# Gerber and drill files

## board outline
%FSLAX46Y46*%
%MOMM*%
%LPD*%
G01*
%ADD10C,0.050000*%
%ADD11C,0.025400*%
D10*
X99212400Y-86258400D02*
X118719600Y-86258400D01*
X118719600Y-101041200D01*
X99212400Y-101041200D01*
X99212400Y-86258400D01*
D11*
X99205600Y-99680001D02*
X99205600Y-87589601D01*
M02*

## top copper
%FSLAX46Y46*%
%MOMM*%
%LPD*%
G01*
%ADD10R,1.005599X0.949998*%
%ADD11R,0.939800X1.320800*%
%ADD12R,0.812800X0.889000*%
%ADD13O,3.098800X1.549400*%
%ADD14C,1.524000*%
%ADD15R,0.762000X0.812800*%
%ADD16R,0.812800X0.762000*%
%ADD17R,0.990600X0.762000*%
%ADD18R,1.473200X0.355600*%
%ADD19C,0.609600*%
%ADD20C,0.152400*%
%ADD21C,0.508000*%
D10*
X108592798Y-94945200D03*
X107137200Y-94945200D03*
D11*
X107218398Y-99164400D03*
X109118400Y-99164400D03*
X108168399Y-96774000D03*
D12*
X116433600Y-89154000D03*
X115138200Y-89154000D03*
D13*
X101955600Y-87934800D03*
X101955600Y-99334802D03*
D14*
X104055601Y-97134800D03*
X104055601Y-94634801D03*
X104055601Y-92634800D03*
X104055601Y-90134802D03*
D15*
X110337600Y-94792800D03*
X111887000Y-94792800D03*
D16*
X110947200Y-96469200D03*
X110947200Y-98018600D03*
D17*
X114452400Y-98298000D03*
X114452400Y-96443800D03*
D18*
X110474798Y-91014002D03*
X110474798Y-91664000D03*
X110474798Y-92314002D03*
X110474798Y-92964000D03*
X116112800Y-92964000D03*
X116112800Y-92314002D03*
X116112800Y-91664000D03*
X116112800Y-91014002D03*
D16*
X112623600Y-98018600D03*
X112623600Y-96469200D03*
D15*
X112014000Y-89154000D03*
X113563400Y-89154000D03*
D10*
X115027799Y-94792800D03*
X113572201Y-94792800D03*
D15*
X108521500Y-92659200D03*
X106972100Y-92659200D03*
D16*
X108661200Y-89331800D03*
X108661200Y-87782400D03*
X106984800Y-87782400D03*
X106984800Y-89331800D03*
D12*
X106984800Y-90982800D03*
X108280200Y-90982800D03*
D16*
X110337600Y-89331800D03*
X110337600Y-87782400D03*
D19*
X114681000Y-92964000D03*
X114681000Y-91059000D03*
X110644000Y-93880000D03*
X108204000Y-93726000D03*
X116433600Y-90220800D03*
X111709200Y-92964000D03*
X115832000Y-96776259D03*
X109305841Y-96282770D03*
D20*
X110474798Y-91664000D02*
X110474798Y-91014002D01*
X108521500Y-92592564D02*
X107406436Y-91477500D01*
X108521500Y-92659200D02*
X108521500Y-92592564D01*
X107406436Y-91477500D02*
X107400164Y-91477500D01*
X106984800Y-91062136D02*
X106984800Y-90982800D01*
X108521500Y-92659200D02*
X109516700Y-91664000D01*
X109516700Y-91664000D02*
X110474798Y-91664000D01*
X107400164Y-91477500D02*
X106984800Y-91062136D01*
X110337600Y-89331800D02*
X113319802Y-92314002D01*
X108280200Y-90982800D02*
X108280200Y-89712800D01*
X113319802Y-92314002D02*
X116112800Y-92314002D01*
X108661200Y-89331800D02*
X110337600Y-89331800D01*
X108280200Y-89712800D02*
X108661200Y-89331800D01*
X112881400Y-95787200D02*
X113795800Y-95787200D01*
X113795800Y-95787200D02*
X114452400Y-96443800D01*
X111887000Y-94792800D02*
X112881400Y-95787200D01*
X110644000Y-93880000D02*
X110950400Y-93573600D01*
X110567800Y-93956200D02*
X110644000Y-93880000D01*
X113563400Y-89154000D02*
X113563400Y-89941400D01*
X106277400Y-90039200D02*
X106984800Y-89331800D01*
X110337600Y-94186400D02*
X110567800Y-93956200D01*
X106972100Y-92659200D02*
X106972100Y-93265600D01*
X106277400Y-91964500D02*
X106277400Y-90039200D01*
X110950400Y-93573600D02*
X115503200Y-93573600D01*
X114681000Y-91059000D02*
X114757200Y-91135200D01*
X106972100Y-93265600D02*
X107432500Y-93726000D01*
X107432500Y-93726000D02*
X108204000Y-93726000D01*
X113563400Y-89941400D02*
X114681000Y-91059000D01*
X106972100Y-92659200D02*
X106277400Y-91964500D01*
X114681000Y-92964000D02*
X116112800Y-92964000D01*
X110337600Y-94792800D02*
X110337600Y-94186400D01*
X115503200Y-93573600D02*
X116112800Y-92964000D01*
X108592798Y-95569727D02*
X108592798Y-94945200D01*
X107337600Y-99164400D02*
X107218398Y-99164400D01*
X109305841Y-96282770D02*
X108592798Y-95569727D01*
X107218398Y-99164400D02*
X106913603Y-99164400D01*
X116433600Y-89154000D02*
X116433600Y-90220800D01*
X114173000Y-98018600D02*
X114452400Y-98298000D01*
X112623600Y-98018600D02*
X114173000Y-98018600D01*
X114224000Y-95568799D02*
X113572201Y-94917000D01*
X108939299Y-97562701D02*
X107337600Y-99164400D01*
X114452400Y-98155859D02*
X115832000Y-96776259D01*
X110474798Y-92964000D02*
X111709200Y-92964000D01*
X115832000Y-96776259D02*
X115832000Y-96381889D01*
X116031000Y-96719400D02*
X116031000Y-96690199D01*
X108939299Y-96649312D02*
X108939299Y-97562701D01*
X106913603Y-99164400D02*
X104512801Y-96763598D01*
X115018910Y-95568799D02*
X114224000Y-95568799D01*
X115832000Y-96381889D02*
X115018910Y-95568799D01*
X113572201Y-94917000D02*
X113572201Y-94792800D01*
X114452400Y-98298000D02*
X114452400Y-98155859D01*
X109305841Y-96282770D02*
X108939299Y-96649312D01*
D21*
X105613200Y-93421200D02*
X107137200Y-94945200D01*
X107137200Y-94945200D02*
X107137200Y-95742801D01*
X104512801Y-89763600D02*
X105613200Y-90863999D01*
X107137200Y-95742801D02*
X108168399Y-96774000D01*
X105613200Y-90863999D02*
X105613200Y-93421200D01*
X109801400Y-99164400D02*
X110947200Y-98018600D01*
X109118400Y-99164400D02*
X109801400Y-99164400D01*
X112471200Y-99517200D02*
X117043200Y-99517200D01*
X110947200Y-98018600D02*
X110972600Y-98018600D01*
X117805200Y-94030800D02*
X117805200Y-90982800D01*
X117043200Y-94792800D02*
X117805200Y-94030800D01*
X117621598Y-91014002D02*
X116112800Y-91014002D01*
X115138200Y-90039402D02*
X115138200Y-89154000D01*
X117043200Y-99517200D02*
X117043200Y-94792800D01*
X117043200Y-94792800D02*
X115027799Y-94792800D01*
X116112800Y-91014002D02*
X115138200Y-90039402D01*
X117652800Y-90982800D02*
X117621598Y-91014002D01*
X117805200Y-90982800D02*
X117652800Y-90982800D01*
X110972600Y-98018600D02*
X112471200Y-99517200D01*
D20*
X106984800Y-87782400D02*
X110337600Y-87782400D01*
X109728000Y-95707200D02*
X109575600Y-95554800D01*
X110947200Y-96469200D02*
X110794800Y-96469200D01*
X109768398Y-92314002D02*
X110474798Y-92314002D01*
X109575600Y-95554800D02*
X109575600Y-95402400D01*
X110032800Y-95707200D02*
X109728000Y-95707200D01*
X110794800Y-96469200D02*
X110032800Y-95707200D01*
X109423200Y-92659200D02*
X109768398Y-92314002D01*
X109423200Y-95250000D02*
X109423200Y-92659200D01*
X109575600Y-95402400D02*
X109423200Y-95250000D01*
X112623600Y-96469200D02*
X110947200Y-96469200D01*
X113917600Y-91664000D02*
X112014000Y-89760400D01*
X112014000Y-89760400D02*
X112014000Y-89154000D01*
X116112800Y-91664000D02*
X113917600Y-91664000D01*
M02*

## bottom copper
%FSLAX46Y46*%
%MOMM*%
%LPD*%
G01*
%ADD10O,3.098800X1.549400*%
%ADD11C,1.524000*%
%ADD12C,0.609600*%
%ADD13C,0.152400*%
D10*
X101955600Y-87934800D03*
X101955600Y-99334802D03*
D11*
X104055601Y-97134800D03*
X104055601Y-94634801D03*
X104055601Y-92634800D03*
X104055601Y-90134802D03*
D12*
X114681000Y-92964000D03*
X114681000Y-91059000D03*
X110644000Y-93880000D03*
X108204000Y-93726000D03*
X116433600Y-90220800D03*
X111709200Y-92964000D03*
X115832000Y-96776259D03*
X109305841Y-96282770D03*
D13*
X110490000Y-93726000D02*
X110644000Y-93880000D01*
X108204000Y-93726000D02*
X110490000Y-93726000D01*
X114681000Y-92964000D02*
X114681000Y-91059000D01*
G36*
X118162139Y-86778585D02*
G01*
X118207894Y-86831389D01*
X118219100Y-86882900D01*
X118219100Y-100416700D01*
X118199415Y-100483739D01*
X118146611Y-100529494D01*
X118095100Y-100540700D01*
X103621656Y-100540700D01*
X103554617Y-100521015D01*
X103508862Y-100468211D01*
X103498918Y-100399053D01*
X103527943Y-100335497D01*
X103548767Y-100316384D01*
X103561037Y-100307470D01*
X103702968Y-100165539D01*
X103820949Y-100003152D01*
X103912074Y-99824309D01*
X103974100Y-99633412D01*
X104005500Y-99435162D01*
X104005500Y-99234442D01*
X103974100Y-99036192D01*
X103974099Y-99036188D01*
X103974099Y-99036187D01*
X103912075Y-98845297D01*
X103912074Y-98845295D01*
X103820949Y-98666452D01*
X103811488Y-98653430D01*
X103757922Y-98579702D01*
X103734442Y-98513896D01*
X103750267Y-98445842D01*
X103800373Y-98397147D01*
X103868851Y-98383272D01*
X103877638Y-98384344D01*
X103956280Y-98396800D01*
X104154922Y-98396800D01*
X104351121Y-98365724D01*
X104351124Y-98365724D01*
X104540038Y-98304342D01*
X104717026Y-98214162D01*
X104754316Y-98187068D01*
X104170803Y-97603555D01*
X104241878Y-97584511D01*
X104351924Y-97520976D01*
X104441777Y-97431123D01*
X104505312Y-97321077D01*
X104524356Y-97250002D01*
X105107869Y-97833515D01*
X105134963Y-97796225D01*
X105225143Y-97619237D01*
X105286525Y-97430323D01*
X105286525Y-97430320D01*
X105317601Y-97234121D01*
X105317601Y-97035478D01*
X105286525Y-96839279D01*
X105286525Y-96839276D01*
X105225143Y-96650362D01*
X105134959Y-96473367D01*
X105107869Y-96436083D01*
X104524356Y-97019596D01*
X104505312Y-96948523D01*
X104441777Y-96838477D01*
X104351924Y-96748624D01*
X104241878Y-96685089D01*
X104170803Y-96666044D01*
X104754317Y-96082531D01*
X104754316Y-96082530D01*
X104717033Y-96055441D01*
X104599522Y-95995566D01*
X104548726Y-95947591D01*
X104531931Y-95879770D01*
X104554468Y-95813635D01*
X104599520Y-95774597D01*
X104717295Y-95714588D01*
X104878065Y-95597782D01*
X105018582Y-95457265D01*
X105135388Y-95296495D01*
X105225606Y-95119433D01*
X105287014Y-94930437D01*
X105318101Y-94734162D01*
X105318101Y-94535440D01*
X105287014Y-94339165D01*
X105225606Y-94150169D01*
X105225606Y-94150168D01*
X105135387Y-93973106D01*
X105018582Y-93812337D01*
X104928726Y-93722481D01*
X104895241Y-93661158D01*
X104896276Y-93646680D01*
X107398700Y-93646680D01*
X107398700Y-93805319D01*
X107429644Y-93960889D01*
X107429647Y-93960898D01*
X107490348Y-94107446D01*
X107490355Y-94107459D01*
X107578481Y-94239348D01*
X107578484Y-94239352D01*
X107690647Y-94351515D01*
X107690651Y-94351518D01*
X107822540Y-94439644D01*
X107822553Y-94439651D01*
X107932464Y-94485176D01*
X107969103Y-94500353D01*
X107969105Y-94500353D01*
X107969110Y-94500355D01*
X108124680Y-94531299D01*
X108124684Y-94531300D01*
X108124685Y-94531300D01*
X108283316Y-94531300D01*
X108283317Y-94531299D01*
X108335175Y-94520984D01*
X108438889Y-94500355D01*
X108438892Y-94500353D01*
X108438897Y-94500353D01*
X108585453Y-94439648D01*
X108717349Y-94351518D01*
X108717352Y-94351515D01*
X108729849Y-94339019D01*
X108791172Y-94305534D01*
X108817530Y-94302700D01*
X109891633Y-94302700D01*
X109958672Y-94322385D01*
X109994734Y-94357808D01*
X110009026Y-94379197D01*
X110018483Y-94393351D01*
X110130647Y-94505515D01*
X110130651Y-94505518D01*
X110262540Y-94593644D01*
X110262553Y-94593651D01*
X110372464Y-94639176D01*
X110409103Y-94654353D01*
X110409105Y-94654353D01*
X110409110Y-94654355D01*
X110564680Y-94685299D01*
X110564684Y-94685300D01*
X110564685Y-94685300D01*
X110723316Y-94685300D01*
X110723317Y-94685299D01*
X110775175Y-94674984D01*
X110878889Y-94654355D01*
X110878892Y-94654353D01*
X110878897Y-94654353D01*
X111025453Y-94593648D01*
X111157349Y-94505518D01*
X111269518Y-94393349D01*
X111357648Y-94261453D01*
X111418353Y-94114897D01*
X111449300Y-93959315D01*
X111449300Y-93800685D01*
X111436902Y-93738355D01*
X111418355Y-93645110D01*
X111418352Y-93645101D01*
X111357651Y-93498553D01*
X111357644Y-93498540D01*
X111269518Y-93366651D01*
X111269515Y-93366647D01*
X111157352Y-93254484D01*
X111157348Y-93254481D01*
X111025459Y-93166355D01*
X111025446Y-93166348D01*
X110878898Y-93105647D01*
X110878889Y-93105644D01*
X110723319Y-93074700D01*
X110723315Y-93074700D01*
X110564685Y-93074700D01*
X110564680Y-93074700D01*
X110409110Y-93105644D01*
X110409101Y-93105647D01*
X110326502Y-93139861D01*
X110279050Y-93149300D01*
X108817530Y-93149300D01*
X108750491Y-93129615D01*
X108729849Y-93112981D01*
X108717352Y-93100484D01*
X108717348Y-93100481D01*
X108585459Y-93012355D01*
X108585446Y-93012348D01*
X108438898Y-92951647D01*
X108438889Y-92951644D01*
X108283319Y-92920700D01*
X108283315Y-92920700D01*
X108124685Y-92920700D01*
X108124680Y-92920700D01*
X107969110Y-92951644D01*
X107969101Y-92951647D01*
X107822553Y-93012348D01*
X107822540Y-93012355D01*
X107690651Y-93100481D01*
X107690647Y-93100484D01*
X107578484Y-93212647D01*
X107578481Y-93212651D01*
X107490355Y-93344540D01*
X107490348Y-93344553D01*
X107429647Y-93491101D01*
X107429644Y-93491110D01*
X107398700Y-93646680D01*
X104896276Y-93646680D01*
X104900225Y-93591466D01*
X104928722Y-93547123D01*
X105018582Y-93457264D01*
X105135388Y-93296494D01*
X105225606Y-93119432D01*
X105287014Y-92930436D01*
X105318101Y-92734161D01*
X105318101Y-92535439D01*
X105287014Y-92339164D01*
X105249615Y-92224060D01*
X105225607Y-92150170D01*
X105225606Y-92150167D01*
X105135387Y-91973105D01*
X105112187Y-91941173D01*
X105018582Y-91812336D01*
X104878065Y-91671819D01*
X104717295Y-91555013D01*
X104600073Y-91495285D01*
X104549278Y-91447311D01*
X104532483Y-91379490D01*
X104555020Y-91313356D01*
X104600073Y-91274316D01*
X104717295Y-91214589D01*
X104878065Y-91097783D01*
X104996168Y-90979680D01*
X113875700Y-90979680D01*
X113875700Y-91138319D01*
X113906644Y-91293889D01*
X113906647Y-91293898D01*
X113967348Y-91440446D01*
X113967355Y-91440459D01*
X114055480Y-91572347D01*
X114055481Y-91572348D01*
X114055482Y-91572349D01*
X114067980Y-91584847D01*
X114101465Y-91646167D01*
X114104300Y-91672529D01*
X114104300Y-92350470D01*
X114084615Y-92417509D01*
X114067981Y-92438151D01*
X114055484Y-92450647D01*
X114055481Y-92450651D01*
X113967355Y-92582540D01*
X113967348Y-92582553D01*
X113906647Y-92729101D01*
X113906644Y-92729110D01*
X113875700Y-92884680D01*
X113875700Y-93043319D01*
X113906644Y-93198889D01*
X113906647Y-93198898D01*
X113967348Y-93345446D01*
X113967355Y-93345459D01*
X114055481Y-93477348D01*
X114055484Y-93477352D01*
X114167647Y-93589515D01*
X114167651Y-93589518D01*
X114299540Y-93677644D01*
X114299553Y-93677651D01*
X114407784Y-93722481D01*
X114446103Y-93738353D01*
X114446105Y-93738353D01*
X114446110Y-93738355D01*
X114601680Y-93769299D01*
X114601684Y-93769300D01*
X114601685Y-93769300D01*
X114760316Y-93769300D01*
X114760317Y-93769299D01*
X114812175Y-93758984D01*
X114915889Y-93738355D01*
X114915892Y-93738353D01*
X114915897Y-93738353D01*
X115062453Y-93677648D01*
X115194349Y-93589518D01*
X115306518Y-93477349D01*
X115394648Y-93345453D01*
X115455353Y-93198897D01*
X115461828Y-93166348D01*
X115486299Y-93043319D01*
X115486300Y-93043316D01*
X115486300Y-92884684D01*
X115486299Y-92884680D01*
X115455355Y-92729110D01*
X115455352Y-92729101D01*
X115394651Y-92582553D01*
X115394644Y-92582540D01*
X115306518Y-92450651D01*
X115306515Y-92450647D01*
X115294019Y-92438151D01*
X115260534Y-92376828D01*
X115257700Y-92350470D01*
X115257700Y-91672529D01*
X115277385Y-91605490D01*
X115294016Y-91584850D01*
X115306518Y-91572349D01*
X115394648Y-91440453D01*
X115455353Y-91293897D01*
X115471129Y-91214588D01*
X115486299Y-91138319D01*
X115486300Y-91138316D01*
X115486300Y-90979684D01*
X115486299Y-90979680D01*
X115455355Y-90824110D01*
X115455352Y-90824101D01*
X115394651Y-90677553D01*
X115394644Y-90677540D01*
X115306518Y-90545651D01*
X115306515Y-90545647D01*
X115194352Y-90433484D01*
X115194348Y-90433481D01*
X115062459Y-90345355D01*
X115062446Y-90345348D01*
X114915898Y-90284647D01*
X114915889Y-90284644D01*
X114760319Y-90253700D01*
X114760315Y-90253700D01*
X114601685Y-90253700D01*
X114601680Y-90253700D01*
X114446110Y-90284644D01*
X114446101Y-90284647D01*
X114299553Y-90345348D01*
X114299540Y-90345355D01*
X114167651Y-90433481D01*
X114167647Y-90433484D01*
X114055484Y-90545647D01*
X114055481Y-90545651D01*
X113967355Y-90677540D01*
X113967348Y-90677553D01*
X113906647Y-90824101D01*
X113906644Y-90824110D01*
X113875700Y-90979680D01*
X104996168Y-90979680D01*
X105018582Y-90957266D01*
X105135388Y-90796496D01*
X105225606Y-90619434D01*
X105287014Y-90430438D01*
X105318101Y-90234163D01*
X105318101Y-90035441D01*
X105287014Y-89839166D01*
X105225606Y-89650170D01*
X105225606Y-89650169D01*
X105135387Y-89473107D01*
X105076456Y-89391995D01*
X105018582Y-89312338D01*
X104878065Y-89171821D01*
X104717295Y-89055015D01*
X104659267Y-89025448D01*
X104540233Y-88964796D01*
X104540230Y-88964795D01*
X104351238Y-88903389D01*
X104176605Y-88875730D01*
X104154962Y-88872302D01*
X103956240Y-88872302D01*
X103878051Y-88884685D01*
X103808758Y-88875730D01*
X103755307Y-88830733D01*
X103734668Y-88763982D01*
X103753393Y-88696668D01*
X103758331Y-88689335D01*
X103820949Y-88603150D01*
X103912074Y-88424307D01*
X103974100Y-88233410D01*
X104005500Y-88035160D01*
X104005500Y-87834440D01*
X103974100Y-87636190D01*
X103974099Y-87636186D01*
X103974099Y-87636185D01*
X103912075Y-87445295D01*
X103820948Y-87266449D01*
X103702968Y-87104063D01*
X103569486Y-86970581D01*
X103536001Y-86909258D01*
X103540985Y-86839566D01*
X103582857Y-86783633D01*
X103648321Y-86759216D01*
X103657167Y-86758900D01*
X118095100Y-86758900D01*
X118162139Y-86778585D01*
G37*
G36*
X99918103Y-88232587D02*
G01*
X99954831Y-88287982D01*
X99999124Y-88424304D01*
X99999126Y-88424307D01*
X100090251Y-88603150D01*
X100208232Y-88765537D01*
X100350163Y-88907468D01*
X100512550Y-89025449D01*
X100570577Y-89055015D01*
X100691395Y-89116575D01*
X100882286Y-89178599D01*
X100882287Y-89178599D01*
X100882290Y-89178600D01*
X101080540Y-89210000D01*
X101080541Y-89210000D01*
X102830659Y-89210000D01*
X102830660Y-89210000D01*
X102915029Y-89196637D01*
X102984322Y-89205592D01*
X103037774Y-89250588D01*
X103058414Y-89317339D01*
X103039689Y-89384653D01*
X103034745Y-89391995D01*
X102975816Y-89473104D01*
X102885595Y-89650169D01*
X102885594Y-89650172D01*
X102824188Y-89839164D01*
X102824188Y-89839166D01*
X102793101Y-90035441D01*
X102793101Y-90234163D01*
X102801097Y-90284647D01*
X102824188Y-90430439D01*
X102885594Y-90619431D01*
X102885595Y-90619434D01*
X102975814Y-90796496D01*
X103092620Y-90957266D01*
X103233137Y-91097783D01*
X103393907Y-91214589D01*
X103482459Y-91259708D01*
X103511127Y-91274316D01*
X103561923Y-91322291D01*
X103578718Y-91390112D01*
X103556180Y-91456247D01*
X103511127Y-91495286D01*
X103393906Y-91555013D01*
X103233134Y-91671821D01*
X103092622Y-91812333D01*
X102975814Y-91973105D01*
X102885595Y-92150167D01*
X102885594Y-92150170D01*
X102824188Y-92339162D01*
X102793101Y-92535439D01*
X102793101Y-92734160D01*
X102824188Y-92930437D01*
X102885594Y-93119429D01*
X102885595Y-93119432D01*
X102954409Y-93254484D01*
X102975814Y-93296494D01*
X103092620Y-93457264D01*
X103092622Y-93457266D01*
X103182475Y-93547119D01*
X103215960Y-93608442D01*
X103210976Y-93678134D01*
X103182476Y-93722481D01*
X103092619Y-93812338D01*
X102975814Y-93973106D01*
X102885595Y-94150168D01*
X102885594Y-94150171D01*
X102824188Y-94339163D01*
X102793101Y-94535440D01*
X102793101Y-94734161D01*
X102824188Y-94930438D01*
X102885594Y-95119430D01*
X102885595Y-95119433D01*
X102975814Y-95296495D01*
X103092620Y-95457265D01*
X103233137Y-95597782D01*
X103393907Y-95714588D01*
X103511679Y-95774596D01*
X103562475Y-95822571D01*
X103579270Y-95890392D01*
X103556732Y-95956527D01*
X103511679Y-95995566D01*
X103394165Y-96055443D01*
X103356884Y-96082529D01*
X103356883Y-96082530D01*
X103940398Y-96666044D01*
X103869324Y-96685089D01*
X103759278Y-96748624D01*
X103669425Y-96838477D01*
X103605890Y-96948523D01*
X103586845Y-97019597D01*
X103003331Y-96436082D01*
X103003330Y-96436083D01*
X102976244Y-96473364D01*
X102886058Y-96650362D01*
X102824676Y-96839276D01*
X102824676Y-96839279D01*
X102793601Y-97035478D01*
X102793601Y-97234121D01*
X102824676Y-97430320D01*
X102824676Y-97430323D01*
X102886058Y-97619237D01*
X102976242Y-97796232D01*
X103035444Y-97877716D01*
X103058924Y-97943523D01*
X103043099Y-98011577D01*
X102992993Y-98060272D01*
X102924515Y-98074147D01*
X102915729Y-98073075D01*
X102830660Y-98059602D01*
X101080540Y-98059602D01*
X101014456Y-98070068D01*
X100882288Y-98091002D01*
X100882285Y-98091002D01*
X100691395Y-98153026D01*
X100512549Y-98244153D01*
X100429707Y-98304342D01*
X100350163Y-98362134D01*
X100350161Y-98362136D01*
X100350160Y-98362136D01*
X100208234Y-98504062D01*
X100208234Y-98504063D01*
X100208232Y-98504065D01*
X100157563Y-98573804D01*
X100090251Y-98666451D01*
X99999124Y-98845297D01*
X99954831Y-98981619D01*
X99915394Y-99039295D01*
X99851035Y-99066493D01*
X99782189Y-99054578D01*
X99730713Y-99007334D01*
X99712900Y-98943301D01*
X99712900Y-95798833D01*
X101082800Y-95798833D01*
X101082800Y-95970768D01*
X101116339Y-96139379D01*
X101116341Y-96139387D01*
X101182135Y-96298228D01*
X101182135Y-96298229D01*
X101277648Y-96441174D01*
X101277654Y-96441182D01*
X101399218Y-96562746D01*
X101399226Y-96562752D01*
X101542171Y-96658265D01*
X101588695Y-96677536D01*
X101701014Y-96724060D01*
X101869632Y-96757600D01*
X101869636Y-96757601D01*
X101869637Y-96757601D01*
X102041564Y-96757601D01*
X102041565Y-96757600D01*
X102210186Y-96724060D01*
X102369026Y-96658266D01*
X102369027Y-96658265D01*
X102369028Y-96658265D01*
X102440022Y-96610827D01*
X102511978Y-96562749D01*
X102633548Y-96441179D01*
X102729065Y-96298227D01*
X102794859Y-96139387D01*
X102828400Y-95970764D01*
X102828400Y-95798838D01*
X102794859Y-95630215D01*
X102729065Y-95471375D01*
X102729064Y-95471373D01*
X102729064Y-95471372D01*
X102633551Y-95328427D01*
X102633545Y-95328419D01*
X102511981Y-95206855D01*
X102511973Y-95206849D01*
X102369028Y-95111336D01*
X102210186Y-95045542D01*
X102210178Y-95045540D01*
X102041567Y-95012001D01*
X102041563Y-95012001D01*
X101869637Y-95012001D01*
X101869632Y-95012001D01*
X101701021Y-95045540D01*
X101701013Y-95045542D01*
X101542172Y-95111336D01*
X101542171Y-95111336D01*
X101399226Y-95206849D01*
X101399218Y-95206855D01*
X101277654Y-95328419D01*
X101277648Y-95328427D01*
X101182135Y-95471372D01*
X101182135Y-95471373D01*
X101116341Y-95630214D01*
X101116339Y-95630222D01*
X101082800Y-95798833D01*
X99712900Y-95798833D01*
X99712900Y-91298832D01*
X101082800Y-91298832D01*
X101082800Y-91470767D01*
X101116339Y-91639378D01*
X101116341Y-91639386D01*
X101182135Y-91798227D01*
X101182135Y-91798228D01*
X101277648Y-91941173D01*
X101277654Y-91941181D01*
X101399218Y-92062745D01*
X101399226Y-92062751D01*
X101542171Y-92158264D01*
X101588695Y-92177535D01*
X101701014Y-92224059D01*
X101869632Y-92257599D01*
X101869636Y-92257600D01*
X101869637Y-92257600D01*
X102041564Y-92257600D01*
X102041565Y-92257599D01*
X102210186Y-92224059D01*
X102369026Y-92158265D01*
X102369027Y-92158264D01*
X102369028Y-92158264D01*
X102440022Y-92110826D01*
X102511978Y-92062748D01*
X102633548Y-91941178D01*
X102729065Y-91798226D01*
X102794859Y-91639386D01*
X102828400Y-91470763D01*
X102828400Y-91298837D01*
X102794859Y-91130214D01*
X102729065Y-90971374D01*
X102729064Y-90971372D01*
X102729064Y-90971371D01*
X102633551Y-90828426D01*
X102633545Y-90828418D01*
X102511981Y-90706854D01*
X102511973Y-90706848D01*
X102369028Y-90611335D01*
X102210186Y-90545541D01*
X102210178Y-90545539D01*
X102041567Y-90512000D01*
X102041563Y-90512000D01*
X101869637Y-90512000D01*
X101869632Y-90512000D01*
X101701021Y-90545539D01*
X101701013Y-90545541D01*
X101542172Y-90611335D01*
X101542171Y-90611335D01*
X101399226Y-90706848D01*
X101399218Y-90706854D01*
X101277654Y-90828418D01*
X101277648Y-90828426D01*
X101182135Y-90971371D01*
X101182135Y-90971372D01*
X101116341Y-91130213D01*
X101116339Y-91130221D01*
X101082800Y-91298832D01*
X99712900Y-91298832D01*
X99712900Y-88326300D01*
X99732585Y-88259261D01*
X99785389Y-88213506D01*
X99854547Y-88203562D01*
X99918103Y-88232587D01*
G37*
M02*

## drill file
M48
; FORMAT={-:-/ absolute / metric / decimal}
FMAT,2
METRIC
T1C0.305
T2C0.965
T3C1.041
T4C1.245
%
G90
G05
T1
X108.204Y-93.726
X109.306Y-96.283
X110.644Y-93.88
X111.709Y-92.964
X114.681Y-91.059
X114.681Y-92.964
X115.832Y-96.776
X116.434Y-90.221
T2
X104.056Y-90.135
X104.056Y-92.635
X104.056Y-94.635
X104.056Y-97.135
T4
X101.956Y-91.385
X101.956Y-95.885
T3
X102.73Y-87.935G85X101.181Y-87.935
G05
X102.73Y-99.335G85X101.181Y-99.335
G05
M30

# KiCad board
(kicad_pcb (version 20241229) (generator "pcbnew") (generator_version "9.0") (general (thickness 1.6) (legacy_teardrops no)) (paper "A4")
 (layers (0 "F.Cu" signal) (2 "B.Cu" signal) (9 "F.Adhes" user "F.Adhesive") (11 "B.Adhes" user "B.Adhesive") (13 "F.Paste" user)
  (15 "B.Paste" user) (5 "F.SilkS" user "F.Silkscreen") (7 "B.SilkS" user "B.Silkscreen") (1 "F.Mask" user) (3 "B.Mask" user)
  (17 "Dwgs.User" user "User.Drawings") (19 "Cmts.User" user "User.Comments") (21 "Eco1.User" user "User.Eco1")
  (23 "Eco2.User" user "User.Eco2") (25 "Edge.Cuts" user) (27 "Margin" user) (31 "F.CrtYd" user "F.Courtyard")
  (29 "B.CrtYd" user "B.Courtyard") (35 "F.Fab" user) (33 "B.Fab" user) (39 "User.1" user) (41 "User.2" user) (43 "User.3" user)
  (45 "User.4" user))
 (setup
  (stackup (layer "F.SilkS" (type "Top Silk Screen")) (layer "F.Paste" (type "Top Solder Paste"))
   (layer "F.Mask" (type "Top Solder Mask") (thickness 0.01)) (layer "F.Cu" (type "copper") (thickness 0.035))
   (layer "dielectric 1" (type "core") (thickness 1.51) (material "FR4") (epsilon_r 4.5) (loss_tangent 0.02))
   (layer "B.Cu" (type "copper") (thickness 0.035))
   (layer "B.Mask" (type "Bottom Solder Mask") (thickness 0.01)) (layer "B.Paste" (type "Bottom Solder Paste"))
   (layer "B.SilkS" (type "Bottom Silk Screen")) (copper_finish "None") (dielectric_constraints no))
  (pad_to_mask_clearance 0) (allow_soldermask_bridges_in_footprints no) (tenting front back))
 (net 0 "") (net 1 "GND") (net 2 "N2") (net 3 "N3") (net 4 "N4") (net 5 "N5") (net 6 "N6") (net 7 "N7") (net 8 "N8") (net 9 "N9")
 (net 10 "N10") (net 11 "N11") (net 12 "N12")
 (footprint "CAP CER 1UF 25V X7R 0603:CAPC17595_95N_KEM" (layer "F.Cu") (at 107.864999 94.9452 180)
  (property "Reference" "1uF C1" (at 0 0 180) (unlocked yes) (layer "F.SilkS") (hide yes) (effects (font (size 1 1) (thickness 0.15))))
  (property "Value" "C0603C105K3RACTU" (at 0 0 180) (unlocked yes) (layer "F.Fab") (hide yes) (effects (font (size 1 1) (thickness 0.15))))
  (pad "1" smd rect (at -0.727799 0 180) (size 1.005599 0.949998) (layers "F.Cu" "F.Mask" "F.Paste") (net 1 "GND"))
  (pad "2" smd rect (at 0.727799 0 180) (size 1.005599 0.949998) (layers "F.Cu" "F.Mask" "F.Paste") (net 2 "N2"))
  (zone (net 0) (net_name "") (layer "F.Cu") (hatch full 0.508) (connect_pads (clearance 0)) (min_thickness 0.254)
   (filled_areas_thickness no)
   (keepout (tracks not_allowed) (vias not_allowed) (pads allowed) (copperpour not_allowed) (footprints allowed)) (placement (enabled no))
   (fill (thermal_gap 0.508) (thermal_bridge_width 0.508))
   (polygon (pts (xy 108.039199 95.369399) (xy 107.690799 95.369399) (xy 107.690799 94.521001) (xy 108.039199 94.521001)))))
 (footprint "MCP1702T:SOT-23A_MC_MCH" (layer "F.Cu") (at 108.168399 97.9692)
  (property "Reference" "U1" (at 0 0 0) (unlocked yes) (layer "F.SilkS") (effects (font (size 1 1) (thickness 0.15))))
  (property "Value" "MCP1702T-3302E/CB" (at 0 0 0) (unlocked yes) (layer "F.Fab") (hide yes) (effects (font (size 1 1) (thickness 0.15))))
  (pad "1" smd rect (at -0.950001 1.1952) (size 0.9398 1.3208) (layers "F.Cu" "F.Mask" "F.Paste") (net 1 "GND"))
  (pad "2" smd rect (at 0.950001 1.1952) (size 0.9398 1.3208) (layers "F.Cu" "F.Mask" "F.Paste") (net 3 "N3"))
  (pad "3" smd rect (at 0 -1.1952) (size 0.9398 1.3208) (layers "F.Cu" "F.Mask" "F.Paste") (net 2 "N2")))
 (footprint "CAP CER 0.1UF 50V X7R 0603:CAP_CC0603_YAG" (layer "F.Cu") (at 115.7859 89.154 180)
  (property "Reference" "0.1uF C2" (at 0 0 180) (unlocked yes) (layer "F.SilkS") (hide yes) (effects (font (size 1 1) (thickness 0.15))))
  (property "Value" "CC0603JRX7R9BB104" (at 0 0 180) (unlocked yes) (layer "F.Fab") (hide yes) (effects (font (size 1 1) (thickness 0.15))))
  (pad "1" smd rect (at -0.6477 0 180) (size 0.8128 0.889) (layers "F.Cu" "F.Mask" "F.Paste") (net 1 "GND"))
  (pad "2" smd rect (at 0.6477 0 180) (size 0.8128 0.889) (layers "F.Cu" "F.Mask" "F.Paste") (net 3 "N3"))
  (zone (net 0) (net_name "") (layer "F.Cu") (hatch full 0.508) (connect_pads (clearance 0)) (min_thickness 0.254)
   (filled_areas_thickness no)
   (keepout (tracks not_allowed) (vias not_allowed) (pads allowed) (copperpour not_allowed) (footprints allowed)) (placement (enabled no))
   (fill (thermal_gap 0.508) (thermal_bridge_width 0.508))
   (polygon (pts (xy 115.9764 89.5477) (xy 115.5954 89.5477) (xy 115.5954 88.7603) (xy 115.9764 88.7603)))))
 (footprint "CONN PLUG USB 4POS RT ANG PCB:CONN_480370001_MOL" (layer "F.Cu") (at 104.055601 97.1348 -90)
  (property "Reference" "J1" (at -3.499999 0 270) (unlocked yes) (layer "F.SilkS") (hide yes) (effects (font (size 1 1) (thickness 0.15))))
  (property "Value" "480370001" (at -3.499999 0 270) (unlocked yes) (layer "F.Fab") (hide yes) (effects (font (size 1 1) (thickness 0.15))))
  (fp_line (start 2.545201 4.850001) (end -9.545199 4.850001) (stroke (width 0.0254) (type solid)) (layer "Edge.Cuts"))
  (pad "" np_thru_hole oval (at -9.2 2.100001 270) (size 1.5494 3.0988) (drill oval 1.0414 2.5908) (layers "*.Cu" "*.Mask"))
  (pad "" np_thru_hole circle (at -5.75 2.100001 270) (size 1.2446 1.2446) (drill 1.2446) (layers))
  (pad "" np_thru_hole circle (at -1.249999 2.100001 270) (size 1.2446 1.2446) (drill 1.2446) (layers))
  (pad "" np_thru_hole oval (at 2.200002 2.100001 270) (size 1.5494 3.0988) (drill oval 1.0414 2.5908) (layers "*.Cu" "*.Mask"))
  (pad "1" thru_hole circle (at 0 0 270) (size 1.524 1.524) (drill 0.9652) (layers "*.Cu" "*.Mask") (remove_unused_layers no) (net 1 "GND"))
  (pad "2" thru_hole circle (at -2.499999 0 270) (size 1.524 1.524) (drill 0.9652) (layers "*.Cu" "*.Mask") (remove_unused_layers no)
   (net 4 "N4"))
  (pad "3" thru_hole circle (at -4.5 0 270) (size 1.524 1.524) (drill 0.9652) (layers "*.Cu" "*.Mask") (remove_unused_layers no)
   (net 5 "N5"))
  (pad "4" thru_hole circle (at -6.999998 0 270) (size 1.524 1.524) (drill 0.9652) (layers "*.Cu" "*.Mask") (remove_unused_layers no)
   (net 2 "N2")))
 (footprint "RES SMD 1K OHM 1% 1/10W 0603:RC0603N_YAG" (layer "F.Cu") (at 111.1123 94.7928)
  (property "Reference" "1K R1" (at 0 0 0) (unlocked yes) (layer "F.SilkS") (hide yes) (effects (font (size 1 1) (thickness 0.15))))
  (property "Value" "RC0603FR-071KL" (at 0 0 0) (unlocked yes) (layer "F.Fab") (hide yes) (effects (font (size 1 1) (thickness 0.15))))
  (pad "1" smd rect (at -0.7747 0) (size 0.762 0.8128) (layers "F.Cu" "F.Mask" "F.Paste") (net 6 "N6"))
  (pad "2" smd rect (at 0.7747 0) (size 0.762 0.8128) (layers "F.Cu" "F.Mask" "F.Paste") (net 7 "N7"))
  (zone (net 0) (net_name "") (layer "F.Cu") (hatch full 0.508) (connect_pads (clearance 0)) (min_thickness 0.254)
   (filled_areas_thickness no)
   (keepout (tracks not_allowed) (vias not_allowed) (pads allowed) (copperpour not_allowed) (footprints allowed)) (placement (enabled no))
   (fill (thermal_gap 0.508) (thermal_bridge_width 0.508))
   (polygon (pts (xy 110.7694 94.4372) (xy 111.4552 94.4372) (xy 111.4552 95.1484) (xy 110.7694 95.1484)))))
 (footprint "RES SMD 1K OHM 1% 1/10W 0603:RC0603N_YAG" (layer "F.Cu") (at 110.9472 97.2439 -90)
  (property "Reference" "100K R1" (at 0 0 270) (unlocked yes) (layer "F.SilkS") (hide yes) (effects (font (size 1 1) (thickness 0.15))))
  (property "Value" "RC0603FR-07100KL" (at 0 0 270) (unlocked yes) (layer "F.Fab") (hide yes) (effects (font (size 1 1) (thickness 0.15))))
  (pad "1" smd rect (at -0.7747 0 270) (size 0.762 0.8128) (layers "F.Cu" "F.Mask" "F.Paste") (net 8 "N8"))
  (pad "2" smd rect (at 0.7747 0 270) (size 0.762 0.8128) (layers "F.Cu" "F.Mask" "F.Paste") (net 3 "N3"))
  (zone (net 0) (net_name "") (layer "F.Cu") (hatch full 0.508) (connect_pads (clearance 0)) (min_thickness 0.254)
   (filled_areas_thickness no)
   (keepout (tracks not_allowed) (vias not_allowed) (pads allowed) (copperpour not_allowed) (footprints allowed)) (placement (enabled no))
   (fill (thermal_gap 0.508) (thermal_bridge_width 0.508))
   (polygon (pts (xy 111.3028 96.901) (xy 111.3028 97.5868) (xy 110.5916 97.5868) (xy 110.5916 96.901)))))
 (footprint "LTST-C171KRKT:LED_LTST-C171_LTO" (layer "F.Cu") (at 114.4524 97.3709 90)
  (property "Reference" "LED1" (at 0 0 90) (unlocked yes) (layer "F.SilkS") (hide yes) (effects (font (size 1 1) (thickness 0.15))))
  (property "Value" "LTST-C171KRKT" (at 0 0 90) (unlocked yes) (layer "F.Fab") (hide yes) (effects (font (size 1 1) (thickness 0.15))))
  (pad "1" smd rect (at -0.9271 0 90) (size 0.762 0.9906) (layers "F.Cu" "F.Mask" "F.Paste") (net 1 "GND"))
  (pad "2" smd rect (at 0.9271 0 90) (size 0.762 0.9906) (layers "F.Cu" "F.Mask" "F.Paste") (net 7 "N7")))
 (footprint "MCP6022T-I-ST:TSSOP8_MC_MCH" (layer "F.Cu") (at 113.293799 91.989001)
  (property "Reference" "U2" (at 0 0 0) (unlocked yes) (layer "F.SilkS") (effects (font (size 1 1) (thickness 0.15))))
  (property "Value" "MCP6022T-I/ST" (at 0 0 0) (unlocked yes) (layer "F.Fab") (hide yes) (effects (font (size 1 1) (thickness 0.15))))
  (pad "1" smd rect (at -2.819001 -0.974999) (size 1.4732 0.3556) (layers "F.Cu" "F.Mask" "F.Paste") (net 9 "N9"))
  (pad "2" smd rect (at -2.819001 -0.325001) (size 1.4732 0.3556) (layers "F.Cu" "F.Mask" "F.Paste") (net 9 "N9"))
  (pad "3" smd rect (at -2.819001 0.325001) (size 1.4732 0.3556) (layers "F.Cu" "F.Mask" "F.Paste") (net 8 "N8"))
  (pad "4" smd rect (at -2.819001 0.974999) (size 1.4732 0.3556) (layers "F.Cu" "F.Mask" "F.Paste") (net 1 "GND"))
  (pad "5" smd rect (at 2.819001 0.974999) (size 1.4732 0.3556) (layers "F.Cu" "F.Mask" "F.Paste") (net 6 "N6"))
  (pad "6" smd rect (at 2.819001 0.325001) (size 1.4732 0.3556) (layers "F.Cu" "F.Mask" "F.Paste") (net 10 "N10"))
  (pad "7" smd rect (at 2.819001 -0.325001) (size 1.4732 0.3556) (layers "F.Cu" "F.Mask" "F.Paste") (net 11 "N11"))
  (pad "8" smd rect (at 2.819001 -0.974999) (size 1.4732 0.3556) (layers "F.Cu" "F.Mask" "F.Paste") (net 3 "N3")))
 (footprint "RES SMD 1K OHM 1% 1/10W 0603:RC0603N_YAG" (layer "F.Cu") (at 112.6236 97.2439 90)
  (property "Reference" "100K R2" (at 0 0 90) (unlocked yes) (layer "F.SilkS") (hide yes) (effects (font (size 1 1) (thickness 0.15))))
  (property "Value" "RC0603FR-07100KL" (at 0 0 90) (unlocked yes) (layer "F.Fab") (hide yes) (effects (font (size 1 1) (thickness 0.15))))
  (pad "1" smd rect (at -0.7747 0 90) (size 0.762 0.8128) (layers "F.Cu" "F.Mask" "F.Paste") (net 1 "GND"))
  (pad "2" smd rect (at 0.7747 0 90) (size 0.762 0.8128) (layers "F.Cu" "F.Mask" "F.Paste") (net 8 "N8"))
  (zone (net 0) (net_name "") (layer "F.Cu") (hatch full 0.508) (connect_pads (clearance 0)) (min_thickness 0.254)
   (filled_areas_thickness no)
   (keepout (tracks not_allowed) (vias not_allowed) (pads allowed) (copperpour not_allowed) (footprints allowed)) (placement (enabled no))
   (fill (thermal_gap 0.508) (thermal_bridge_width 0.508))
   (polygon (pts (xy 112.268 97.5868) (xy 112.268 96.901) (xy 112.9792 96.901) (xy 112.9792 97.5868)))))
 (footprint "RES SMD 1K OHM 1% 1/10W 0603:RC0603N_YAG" (layer "F.Cu") (at 112.7887 89.154)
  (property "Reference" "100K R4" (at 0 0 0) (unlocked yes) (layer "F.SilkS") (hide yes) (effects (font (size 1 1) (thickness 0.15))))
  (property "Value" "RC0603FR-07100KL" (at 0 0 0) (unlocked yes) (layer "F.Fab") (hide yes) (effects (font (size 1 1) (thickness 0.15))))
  (pad "1" smd rect (at -0.7747 0) (size 0.762 0.8128) (layers "F.Cu" "F.Mask" "F.Paste") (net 11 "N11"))
  (pad "2" smd rect (at 0.7747 0) (size 0.762 0.8128) (layers "F.Cu" "F.Mask" "F.Paste") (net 6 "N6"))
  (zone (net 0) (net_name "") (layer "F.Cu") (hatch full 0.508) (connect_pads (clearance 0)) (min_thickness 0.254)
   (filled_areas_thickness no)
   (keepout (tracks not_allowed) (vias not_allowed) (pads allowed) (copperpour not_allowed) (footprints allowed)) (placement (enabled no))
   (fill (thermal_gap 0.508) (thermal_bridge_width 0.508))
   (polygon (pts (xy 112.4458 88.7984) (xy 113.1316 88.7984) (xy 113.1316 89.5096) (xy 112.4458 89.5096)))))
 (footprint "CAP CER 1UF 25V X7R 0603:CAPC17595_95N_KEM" (layer "F.Cu") (at 114.3 94.7928 180)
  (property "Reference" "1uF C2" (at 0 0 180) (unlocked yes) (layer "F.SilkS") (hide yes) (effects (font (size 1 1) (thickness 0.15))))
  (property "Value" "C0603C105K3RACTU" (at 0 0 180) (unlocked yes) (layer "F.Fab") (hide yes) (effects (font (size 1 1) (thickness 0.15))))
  (pad "1" smd rect (at -0.727799 0 180) (size 1.005599 0.949998) (layers "F.Cu" "F.Mask" "F.Paste") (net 3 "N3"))
  (pad "2" smd rect (at 0.727799 0 180) (size 1.005599 0.949998) (layers "F.Cu" "F.Mask" "F.Paste") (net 1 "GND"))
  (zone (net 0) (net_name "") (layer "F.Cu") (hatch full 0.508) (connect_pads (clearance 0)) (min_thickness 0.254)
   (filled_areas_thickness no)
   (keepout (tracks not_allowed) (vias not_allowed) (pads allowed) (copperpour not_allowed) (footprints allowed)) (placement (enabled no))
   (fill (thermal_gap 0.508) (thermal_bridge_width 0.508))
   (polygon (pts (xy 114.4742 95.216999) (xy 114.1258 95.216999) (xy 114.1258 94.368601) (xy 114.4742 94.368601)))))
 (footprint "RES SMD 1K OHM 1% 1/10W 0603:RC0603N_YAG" (layer "F.Cu") (at 107.7468 92.6592 180)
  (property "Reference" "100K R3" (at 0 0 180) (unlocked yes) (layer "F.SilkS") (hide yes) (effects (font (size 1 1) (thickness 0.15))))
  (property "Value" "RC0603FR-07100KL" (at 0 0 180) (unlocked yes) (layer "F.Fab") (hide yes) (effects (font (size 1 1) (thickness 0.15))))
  (pad "1" smd rect (at -0.7747 0 180) (size 0.762 0.8128) (layers "F.Cu" "F.Mask" "F.Paste") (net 9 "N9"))
  (pad "2" smd rect (at 0.7747 0 180) (size 0.762 0.8128) (layers "F.Cu" "F.Mask" "F.Paste") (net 6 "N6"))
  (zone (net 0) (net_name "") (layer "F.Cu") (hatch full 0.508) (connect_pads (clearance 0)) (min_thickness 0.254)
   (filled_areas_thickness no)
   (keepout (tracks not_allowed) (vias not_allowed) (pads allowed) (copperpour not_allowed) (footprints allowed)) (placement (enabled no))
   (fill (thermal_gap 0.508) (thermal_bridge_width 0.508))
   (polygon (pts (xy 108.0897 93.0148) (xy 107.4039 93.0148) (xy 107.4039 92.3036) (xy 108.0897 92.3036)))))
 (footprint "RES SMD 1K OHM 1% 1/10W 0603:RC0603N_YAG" (layer "F.Cu") (at 108.6612 88.5571 90)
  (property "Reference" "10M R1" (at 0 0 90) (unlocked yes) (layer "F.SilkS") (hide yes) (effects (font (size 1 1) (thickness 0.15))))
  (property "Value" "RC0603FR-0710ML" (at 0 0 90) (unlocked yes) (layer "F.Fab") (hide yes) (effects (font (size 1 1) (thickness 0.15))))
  (pad "1" smd rect (at -0.7747 0 90) (size 0.762 0.8128) (layers "F.Cu" "F.Mask" "F.Paste") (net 10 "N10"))
  (pad "2" smd rect (at 0.7747 0 90) (size 0.762 0.8128) (layers "F.Cu" "F.Mask" "F.Paste") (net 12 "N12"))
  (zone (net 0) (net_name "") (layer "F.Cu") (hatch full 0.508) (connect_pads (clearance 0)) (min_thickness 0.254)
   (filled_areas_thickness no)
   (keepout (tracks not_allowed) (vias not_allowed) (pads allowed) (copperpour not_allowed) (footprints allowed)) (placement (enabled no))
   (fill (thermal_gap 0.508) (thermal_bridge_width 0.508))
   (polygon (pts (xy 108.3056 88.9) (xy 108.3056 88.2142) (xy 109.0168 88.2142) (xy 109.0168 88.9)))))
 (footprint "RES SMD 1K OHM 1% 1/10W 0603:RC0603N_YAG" (layer "F.Cu") (at 106.9848 88.5571 -90)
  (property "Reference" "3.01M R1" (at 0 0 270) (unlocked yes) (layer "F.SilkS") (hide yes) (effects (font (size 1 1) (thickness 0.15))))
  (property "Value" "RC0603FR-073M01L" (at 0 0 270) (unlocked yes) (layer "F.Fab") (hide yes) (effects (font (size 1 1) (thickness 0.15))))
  (pad "1" smd rect (at -0.7747 0 270) (size 0.762 0.8128) (layers "F.Cu" "F.Mask" "F.Paste") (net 12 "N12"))
  (pad "2" smd rect (at 0.7747 0 270) (size 0.762 0.8128) (layers "F.Cu" "F.Mask" "F.Paste") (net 6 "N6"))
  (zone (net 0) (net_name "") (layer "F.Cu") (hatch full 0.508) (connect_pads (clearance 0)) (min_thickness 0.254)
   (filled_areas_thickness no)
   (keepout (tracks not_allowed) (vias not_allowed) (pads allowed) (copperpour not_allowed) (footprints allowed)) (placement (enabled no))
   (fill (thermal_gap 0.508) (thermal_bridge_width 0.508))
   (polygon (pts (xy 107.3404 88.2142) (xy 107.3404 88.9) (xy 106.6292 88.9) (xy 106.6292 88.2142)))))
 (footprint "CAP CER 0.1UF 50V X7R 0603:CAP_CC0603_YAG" (layer "F.Cu") (at 107.6325 90.9828)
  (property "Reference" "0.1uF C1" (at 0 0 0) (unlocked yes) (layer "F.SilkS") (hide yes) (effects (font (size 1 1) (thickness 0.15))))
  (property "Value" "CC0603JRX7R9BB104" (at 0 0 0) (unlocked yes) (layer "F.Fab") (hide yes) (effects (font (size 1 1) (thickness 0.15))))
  (pad "1" smd rect (at -0.6477 0) (size 0.8128 0.889) (layers "F.Cu" "F.Mask" "F.Paste") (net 9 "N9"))
  (pad "2" smd rect (at 0.6477 0) (size 0.8128 0.889) (layers "F.Cu" "F.Mask" "F.Paste") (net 10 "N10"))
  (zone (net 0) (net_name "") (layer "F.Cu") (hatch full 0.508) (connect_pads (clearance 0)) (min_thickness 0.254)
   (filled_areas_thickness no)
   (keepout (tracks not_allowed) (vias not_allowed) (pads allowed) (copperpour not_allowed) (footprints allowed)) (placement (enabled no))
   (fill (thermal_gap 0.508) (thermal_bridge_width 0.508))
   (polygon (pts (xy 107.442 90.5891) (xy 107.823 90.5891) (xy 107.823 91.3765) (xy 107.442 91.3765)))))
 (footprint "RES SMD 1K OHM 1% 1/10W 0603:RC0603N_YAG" (layer "F.Cu") (at 110.3376 88.5571 90)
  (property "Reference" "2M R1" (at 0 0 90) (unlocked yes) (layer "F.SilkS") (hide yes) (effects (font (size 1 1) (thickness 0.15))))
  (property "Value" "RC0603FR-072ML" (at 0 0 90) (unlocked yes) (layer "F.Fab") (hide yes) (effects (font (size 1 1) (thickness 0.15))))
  (pad "1" smd rect (at -0.7747 0 90) (size 0.762 0.8128) (layers "F.Cu" "F.Mask" "F.Paste") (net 10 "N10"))
  (pad "2" smd rect (at 0.7747 0 90) (size 0.762 0.8128) (layers "F.Cu" "F.Mask" "F.Paste") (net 12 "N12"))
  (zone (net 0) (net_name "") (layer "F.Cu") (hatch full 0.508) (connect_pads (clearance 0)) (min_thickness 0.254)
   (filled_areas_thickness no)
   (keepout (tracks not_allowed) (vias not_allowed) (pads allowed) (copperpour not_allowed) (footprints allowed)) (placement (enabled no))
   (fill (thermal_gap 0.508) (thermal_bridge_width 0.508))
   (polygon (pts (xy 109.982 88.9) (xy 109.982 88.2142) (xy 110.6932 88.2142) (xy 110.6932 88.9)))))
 (gr_rect (start 99.2124 86.2584) (end 118.7196 101.0412) (stroke (width 0.05) (type default)) (fill no) (layer "Edge.Cuts"))
 (segment (start 110.474798 91.664) (end 110.474798 91.014002) (width 0.1524) (layer "F.Cu") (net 9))
 (segment (start 108.5215 92.592564) (end 107.406436 91.4775) (width 0.1524) (layer "F.Cu") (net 9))
 (segment (start 108.5215 92.6592) (end 108.5215 92.592564) (width 0.1524) (layer "F.Cu") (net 9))
 (segment (start 107.406436 91.4775) (end 107.400164 91.4775) (width 0.1524) (layer "F.Cu") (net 9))
 (segment (start 106.9848 91.062136) (end 106.9848 90.9828) (width 0.1524) (layer "F.Cu") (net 9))
 (segment (start 108.5215 92.6592) (end 109.5167 91.664) (width 0.1524) (layer "F.Cu") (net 9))
 (segment (start 109.5167 91.664) (end 110.474798 91.664) (width 0.1524) (layer "F.Cu") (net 9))
 (segment (start 107.400164 91.4775) (end 106.9848 91.062136) (width 0.1524) (layer "F.Cu") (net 9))
 (segment (start 110.3376 89.3318) (end 113.319802 92.314002) (width 0.1524) (layer "F.Cu") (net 10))
 (segment (start 108.2802 90.9828) (end 108.2802 89.7128) (width 0.1524) (layer "F.Cu") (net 10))
 (segment (start 113.319802 92.314002) (end 116.1128 92.314002) (width 0.1524) (layer "F.Cu") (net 10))
 (segment (start 108.6612 89.3318) (end 110.3376 89.3318) (width 0.1524) (layer "F.Cu") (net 10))
 (segment (start 108.2802 89.7128) (end 108.6612 89.3318) (width 0.1524) (layer "F.Cu") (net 10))
 (segment (start 112.8814 95.7872) (end 113.7958 95.7872) (width 0.1524) (layer "F.Cu") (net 7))
 (segment (start 113.7958 95.7872) (end 114.4524 96.4438) (width 0.1524) (layer "F.Cu") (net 7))
 (segment (start 111.887 94.7928) (end 112.8814 95.7872) (width 0.1524) (layer "F.Cu") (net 7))
 (segment (start 110.644 93.88) (end 110.9504 93.5736) (width 0.1524) (layer "F.Cu") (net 6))
 (segment (start 110.5678 93.9562) (end 110.644 93.88) (width 0.1524) (layer "F.Cu") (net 6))
 (segment (start 113.5634 89.154) (end 113.5634 89.9414) (width 0.1524) (layer "F.Cu") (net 6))
 (segment (start 106.2774 90.0392) (end 106.9848 89.3318) (width 0.1524) (layer "F.Cu") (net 6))
 (segment (start 110.3376 94.1864) (end 110.5678 93.9562) (width 0.1524) (layer "F.Cu") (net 6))
 (segment (start 106.9721 92.6592) (end 106.9721 93.2656) (width 0.1524) (layer "F.Cu") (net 6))
 (segment (start 106.2774 91.9645) (end 106.2774 90.0392) (width 0.1524) (layer "F.Cu") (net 6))
 (segment (start 110.9504 93.5736) (end 115.5032 93.5736) (width 0.1524) (layer "F.Cu") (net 6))
 (segment (start 114.681 91.059) (end 114.7572 91.1352) (width 0.1524) (layer "F.Cu") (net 6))
 (segment (start 106.9721 93.2656) (end 107.4325 93.726) (width 0.1524) (layer "F.Cu") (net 6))
 (segment (start 107.4325 93.726) (end 108.204 93.726) (width 0.1524) (layer "F.Cu") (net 6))
 (segment (start 113.5634 89.9414) (end 114.681 91.059) (width 0.1524) (layer "F.Cu") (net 6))
 (segment (start 106.9721 92.6592) (end 106.2774 91.9645) (width 0.1524) (layer "F.Cu") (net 6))
 (segment (start 114.681 92.964) (end 116.1128 92.964) (width 0.1524) (layer "F.Cu") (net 6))
 (segment (start 110.3376 94.7928) (end 110.3376 94.1864) (width 0.1524) (layer "F.Cu") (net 6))
 (segment (start 115.5032 93.5736) (end 116.1128 92.964) (width 0.1524) (layer "F.Cu") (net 6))
 (via (at 114.681 92.964) (size 0.6096) (drill 0.3048) (layers "F.Cu" "B.Cu") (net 6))
 (via (at 114.681 91.059) (size 0.6096) (drill 0.3048) (layers "F.Cu" "B.Cu") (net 6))
 (via (at 110.644 93.88) (size 0.6096) (drill 0.3048) (layers "F.Cu" "B.Cu") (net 6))
 (via (at 108.204 93.726) (size 0.6096) (drill 0.3048) (layers "F.Cu" "B.Cu") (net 6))
 (segment (start 110.49 93.726) (end 110.644 93.88) (width 0.1524) (layer "B.Cu") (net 6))
 (segment (start 108.204 93.726) (end 110.49 93.726) (width 0.1524) (layer "B.Cu") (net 6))
 (segment (start 114.681 92.964) (end 114.681 91.059) (width 0.1524) (layer "B.Cu") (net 6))
 (segment (start 108.592798 95.569727) (end 108.592798 94.9452) (width 0.1524) (layer "F.Cu") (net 1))
 (segment (start 107.3376 99.1644) (end 107.218398 99.1644) (width 0.1524) (layer "F.Cu") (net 1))
 (segment (start 109.305841 96.28277) (end 108.592798 95.569727) (width 0.1524) (layer "F.Cu") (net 1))
 (segment (start 107.218398 99.1644) (end 106.913603 99.1644) (width 0.1524) (layer "F.Cu") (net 1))
 (segment (start 116.4336 89.154) (end 116.4336 90.2208) (width 0.1524) (layer "F.Cu") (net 1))
 (segment (start 114.173 98.0186) (end 114.4524 98.298) (width 0.1524) (layer "F.Cu") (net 1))
 (segment (start 112.6236 98.0186) (end 114.173 98.0186) (width 0.1524) (layer "F.Cu") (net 1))
 (segment (start 114.224 95.568799) (end 113.572201 94.917) (width 0.1524) (layer "F.Cu") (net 1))
 (segment (start 108.939299 97.562701) (end 107.3376 99.1644) (width 0.1524) (layer "F.Cu") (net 1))
 (segment (start 114.4524 98.155859) (end 115.832 96.776259) (width 0.1524) (layer "F.Cu") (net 1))
 (segment (start 110.474798 92.964) (end 111.7092 92.964) (width 0.1524) (layer "F.Cu") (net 1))
 (segment (start 115.832 96.776259) (end 115.832 96.381889) (width 0.1524) (layer "F.Cu") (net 1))
 (segment (start 116.031 96.7194) (end 116.031 96.690199) (width 0.1524) (layer "F.Cu") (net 1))
 (segment (start 108.939299 96.649312) (end 108.939299 97.562701) (width 0.1524) (layer "F.Cu") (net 1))
 (segment (start 106.913603 99.1644) (end 104.512801 96.763598) (width 0.1524) (layer "F.Cu") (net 1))
 (segment (start 115.01891 95.568799) (end 114.224 95.568799) (width 0.1524) (layer "F.Cu") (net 1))
 (segment (start 115.832 96.381889) (end 115.01891 95.568799) (width 0.1524) (layer "F.Cu") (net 1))
 (segment (start 113.572201 94.917) (end 113.572201 94.7928) (width 0.1524) (layer "F.Cu") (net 1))
 (segment (start 114.4524 98.298) (end 114.4524 98.155859) (width 0.1524) (layer "F.Cu") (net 1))
 (segment (start 109.305841 96.28277) (end 108.939299 96.649312) (width 0.1524) (layer "F.Cu") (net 1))
 (via (at 116.4336 90.2208) (size 0.6096) (drill 0.3048) (layers "F.Cu" "B.Cu") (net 1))
 (via (at 111.7092 92.964) (size 0.6096) (drill 0.3048) (layers "F.Cu" "B.Cu") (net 1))
 (via (at 115.832 96.776259) (size 0.6096) (drill 0.3048) (layers "F.Cu" "B.Cu") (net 1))
 (via (at 109.305841 96.28277) (size 0.6096) (drill 0.3048) (layers "F.Cu" "B.Cu") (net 1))
 (segment (start 105.6132 93.4212) (end 107.1372 94.9452) (width 0.508) (layer "F.Cu") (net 2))
 (segment (start 107.1372 94.9452) (end 107.1372 95.742801) (width 0.508) (layer "F.Cu") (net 2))
 (segment (start 104.512801 89.7636) (end 105.6132 90.863999) (width 0.508) (layer "F.Cu") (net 2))
 (segment (start 107.1372 95.742801) (end 108.168399 96.774) (width 0.508) (layer "F.Cu") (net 2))
 (segment (start 105.6132 90.863999) (end 105.6132 93.4212) (width 0.508) (layer "F.Cu") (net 2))
 (segment (start 109.8014 99.1644) (end 110.9472 98.0186) (width 0.508) (layer "F.Cu") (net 3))
 (segment (start 109.1184 99.1644) (end 109.8014 99.1644) (width 0.508) (layer "F.Cu") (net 3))
 (segment (start 112.4712 99.5172) (end 117.0432 99.5172) (width 0.508) (layer "F.Cu") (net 3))
 (segment (start 110.9472 98.0186) (end 110.9726 98.0186) (width 0.508) (layer "F.Cu") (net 3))
 (segment (start 117.8052 94.0308) (end 117.8052 90.9828) (width 0.508) (layer "F.Cu") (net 3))
 (segment (start 117.0432 94.7928) (end 117.8052 94.0308) (width 0.508) (layer "F.Cu") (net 3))
 (segment (start 117.621598 91.014002) (end 116.1128 91.014002) (width 0.508) (layer "F.Cu") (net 3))
 (segment (start 115.1382 90.039402) (end 115.1382 89.154) (width 0.508) (layer "F.Cu") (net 3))
 (segment (start 117.0432 99.5172) (end 117.0432 94.7928) (width 0.508) (layer "F.Cu") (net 3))
 (segment (start 117.0432 94.7928) (end 115.027799 94.7928) (width 0.508) (layer "F.Cu") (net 3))
 (segment (start 116.1128 91.014002) (end 115.1382 90.039402) (width 0.508) (layer "F.Cu") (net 3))
 (segment (start 117.6528 90.9828) (end 117.621598 91.014002) (width 0.508) (layer "F.Cu") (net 3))
 (segment (start 117.8052 90.9828) (end 117.6528 90.9828) (width 0.508) (layer "F.Cu") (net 3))
 (segment (start 110.9726 98.0186) (end 112.4712 99.5172) (width 0.508) (layer "F.Cu") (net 3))
 (segment (start 106.9848 87.7824) (end 110.3376 87.7824) (width 0.1524) (layer "F.Cu") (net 12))
 (segment (start 109.728 95.7072) (end 109.5756 95.5548) (width 0.1524) (layer "F.Cu") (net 8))
 (segment (start 110.9472 96.4692) (end 110.7948 96.4692) (width 0.1524) (layer "F.Cu") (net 8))
 (segment (start 109.768398 92.314002) (end 110.474798 92.314002) (width 0.1524) (layer "F.Cu") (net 8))
 (segment (start 109.5756 95.5548) (end 109.5756 95.4024) (width 0.1524) (layer "F.Cu") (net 8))
 (segment (start 110.0328 95.7072) (end 109.728 95.7072) (width 0.1524) (layer "F.Cu") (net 8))
 (segment (start 110.7948 96.4692) (end 110.0328 95.7072) (width 0.1524) (layer "F.Cu") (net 8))
 (segment (start 109.4232 92.6592) (end 109.768398 92.314002) (width 0.1524) (layer "F.Cu") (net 8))
 (segment (start 109.4232 95.25) (end 109.4232 92.6592) (width 0.1524) (layer "F.Cu") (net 8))
 (segment (start 109.5756 95.4024) (end 109.4232 95.25) (width 0.1524) (layer "F.Cu") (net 8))
 (segment (start 112.6236 96.4692) (end 110.9472 96.4692) (width 0.1524) (layer "F.Cu") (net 8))
 (segment (start 113.9176 91.664) (end 112.014 89.7604) (width 0.1524) (layer "F.Cu") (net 11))
 (segment (start 112.014 89.7604) (end 112.014 89.154) (width 0.1524) (layer "F.Cu") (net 11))
 (segment (start 116.1128 91.664) (end 113.9176 91.664) (width 0.1524) (layer "F.Cu") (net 11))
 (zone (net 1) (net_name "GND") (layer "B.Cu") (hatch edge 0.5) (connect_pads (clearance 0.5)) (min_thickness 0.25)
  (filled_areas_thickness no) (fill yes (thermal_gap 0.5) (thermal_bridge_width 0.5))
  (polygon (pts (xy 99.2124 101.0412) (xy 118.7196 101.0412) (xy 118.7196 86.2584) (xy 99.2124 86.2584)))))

